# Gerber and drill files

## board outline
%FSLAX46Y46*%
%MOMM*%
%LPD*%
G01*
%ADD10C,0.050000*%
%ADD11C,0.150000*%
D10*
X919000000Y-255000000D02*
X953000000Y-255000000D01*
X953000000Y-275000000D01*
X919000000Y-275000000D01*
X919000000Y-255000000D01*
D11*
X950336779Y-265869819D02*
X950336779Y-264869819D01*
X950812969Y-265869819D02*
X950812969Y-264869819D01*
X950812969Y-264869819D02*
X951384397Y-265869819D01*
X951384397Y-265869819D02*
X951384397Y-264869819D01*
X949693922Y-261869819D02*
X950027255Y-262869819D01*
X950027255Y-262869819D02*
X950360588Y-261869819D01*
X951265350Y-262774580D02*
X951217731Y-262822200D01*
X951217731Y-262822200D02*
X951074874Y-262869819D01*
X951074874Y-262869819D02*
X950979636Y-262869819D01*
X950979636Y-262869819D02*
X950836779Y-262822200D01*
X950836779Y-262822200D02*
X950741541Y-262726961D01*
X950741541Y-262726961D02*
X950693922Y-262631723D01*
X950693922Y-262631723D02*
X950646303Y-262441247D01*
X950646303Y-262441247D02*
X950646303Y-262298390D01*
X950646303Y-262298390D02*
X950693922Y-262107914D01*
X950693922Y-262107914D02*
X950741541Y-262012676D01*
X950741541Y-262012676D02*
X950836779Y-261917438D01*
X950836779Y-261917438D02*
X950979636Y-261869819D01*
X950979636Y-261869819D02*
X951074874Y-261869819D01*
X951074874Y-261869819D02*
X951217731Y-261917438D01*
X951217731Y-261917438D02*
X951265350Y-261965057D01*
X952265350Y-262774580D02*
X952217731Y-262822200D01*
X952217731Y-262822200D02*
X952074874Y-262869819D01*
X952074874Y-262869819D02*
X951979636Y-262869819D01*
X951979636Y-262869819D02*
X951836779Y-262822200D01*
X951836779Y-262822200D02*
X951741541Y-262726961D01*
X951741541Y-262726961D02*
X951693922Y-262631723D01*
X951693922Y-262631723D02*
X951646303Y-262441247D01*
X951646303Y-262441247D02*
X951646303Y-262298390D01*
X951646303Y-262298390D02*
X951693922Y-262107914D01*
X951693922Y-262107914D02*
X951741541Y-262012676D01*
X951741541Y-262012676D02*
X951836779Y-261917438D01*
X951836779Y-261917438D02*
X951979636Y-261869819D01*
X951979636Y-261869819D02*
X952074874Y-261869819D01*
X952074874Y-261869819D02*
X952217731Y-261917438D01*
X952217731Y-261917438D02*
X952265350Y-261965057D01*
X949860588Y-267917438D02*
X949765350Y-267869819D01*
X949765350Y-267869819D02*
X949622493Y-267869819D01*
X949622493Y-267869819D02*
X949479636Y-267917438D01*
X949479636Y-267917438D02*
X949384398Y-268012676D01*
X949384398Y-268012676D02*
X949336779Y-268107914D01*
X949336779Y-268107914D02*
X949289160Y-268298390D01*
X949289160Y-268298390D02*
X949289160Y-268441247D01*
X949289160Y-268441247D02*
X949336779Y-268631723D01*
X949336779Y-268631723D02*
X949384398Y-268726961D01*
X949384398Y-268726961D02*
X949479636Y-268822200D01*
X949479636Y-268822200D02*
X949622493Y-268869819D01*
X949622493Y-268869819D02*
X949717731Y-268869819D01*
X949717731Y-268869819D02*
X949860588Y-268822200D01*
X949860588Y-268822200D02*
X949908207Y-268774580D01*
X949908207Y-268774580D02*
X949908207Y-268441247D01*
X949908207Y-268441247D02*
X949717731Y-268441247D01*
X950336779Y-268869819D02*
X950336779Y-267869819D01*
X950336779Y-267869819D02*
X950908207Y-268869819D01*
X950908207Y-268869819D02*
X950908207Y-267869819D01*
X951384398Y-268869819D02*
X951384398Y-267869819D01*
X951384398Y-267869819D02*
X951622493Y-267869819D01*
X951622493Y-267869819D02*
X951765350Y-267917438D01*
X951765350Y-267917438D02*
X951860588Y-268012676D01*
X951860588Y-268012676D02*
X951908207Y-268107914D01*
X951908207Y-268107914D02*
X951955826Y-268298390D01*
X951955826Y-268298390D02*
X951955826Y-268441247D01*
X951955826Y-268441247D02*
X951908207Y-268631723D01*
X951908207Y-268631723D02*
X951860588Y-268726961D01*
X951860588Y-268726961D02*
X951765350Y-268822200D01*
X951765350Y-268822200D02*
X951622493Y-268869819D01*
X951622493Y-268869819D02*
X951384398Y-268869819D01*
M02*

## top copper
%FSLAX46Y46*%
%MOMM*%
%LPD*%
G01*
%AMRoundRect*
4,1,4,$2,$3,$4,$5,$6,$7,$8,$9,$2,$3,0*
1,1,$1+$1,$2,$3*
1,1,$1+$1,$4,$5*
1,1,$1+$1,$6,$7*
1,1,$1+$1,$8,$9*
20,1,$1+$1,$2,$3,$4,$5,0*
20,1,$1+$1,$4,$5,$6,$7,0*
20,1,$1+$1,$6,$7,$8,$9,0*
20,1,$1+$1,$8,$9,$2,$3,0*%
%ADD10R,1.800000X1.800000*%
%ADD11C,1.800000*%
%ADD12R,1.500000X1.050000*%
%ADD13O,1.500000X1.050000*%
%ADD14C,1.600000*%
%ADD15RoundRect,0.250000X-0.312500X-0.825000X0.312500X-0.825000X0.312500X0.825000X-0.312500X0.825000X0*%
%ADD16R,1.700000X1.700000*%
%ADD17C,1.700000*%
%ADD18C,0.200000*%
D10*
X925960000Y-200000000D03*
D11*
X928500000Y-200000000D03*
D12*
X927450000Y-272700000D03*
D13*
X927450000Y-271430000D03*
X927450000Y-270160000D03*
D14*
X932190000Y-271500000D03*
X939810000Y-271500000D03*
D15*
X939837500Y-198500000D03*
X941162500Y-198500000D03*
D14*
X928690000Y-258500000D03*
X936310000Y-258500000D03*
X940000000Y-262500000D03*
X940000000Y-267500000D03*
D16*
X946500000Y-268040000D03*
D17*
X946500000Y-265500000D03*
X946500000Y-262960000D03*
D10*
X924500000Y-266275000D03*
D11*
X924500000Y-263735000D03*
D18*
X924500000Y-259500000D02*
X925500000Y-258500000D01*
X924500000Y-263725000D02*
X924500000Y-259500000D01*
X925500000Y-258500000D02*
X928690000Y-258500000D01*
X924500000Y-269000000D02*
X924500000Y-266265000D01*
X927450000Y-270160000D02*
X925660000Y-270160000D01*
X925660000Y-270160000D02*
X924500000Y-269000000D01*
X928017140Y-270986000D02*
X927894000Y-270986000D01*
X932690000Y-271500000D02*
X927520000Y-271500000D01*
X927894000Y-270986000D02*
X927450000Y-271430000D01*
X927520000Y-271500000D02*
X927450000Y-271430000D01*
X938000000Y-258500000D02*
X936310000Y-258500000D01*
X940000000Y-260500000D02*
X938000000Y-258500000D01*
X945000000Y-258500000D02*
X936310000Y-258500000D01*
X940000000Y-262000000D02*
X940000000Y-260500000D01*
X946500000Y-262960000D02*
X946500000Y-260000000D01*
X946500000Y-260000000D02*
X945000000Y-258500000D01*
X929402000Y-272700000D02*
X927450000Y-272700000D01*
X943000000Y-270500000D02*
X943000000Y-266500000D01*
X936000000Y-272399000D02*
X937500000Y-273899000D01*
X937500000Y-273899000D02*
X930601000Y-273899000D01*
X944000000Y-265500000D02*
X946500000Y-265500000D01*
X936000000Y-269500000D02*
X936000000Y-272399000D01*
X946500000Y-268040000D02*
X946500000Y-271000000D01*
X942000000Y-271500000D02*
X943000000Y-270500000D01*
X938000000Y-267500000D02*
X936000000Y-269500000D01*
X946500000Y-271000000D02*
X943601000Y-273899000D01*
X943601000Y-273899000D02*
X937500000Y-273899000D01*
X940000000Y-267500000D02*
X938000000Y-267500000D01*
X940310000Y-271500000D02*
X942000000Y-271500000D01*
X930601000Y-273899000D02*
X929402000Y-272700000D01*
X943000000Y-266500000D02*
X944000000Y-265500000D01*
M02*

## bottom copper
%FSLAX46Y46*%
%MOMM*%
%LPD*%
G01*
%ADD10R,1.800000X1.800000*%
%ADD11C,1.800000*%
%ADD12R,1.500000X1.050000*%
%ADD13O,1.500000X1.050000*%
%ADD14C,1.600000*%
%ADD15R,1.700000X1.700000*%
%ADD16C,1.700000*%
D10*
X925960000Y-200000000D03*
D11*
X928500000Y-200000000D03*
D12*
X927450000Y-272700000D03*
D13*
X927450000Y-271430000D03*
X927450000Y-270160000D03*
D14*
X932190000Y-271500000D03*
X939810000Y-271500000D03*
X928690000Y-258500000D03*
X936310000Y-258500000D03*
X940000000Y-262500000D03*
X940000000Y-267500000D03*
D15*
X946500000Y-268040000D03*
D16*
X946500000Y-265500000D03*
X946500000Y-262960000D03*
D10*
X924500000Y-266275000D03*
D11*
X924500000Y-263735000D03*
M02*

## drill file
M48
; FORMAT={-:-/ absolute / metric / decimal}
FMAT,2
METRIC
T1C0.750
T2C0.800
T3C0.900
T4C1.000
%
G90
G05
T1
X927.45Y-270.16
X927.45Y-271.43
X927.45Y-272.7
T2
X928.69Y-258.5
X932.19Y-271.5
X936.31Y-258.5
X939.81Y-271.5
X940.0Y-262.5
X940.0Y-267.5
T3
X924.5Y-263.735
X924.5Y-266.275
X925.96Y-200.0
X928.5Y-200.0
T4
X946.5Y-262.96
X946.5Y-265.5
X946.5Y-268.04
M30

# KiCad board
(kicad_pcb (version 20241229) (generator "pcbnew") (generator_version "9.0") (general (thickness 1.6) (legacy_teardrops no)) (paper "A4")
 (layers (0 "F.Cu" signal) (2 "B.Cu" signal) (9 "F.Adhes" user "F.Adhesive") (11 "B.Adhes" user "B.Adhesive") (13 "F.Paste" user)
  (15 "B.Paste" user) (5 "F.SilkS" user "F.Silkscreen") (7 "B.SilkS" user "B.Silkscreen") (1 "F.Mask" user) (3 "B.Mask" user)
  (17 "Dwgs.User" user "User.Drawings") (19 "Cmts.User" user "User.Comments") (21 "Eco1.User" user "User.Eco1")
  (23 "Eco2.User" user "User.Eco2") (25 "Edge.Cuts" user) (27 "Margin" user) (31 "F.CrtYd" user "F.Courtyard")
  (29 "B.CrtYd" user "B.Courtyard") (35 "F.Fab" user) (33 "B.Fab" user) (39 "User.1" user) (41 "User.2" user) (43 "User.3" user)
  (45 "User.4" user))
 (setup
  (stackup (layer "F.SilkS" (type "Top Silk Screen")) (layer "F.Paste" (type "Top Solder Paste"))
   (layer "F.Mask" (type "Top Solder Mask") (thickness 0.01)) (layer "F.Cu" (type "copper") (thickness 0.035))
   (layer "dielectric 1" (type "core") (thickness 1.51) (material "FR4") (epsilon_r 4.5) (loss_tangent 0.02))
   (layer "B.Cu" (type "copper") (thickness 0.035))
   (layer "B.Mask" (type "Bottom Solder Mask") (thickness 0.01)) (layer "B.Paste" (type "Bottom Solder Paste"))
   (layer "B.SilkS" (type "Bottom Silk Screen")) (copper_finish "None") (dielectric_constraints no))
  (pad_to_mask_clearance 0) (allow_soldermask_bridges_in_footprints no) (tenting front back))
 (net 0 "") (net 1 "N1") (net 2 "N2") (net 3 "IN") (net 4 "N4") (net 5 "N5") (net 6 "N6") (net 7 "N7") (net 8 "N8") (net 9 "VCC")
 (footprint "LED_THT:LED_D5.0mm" (layer "F.Cu") (at 925.96 200)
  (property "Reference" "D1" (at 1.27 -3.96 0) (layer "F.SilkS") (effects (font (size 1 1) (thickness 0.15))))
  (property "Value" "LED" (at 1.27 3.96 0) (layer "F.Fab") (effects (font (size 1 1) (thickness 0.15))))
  (pad "1" thru_hole rect (at 0 0) (size 1.8 1.8) (drill 0.9) (layers "*.Cu" "*.Mask") (remove_unused_layers no) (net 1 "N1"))
  (pad "2" thru_hole circle (at 2.54 0) (size 1.8 1.8) (drill 0.9) (layers "*.Cu" "*.Mask") (remove_unused_layers no) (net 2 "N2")))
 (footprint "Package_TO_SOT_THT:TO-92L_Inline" (layer "F.Cu") (at 927.45 272.7 90)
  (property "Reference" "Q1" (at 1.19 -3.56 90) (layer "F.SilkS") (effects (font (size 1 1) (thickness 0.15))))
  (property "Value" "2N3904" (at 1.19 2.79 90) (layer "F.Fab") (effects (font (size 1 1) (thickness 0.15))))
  (pad "1" thru_hole rect (at 0 0 90) (size 1.05 1.5) (drill 0.75) (layers "*.Cu" "*.Mask") (remove_unused_layers no) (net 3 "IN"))
  (pad "2" thru_hole oval (at 1.27 0 90) (size 1.05 1.5) (drill 0.75) (layers "*.Cu" "*.Mask") (remove_unused_layers no) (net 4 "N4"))
  (pad "3" thru_hole oval (at 2.54 0 90) (size 1.05 1.5) (drill 0.75) (layers "*.Cu" "*.Mask") (remove_unused_layers no) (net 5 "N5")))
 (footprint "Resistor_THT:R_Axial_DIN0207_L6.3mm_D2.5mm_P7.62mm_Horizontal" (layer "F.Cu") (at 932.19 271.5)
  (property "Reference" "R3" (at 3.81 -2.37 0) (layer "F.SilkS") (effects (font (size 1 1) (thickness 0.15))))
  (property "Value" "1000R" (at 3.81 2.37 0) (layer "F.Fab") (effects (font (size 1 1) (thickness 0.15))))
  (pad "1" thru_hole circle (at 0 0) (size 1.6 1.6) (drill 0.8) (layers "*.Cu" "*.Mask") (remove_unused_layers no) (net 4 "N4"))
  (pad "2" thru_hole circle (at 7.62 0) (size 1.6 1.6) (drill 0.8) (layers "*.Cu" "*.Mask") (remove_unused_layers no) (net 3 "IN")))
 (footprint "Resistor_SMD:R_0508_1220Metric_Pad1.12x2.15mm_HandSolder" (layer "F.Cu") (at 940.5 198.5)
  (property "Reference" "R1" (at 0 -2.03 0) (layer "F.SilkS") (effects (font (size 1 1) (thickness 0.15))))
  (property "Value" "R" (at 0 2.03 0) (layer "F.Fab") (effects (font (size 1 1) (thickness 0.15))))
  (pad "1" smd roundrect (at -0.6625 0) (size 1.125 2.15) (layers "F.Cu" "F.Mask" "F.Paste") (roundrect_rratio 0.222222) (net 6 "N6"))
  (pad "2" smd roundrect (at 0.6625 0) (size 1.125 2.15) (layers "F.Cu" "F.Mask" "F.Paste") (roundrect_rratio 0.222222) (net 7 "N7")))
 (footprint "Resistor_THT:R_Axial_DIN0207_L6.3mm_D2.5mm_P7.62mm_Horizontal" (layer "F.Cu") (at 928.69 258.5)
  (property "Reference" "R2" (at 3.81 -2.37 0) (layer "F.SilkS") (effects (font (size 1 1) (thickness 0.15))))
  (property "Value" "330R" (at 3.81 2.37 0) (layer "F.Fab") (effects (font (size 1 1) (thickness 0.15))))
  (pad "1" thru_hole circle (at 0 0) (size 1.6 1.6) (drill 0.8) (layers "*.Cu" "*.Mask") (remove_unused_layers no) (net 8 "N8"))
  (pad "2" thru_hole circle (at 7.62 0) (size 1.6 1.6) (drill 0.8) (layers "*.Cu" "*.Mask") (remove_unused_layers no) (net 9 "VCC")))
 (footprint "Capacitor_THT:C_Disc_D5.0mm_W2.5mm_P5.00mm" (layer "F.Cu") (at 940 262.5 -90)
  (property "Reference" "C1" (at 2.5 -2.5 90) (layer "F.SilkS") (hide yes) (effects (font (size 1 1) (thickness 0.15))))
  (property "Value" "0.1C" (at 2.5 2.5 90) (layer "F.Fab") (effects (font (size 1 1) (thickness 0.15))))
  (pad "1" thru_hole circle (at 0 0 270) (size 1.6 1.6) (drill 0.8) (layers "*.Cu" "*.Mask") (remove_unused_layers no) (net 9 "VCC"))
  (pad "2" thru_hole circle (at 5 0 270) (size 1.6 1.6) (drill 0.8) (layers "*.Cu" "*.Mask") (remove_unused_layers no) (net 3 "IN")))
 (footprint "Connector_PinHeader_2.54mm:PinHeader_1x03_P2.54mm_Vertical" (layer "F.Cu") (at 946.5 268.04 180)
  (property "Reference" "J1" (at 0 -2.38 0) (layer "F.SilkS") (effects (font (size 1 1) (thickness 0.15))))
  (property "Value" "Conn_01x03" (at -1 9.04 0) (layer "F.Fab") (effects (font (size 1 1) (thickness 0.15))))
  (pad "1" thru_hole rect (at 0 0 180) (size 1.7 1.7) (drill 1) (layers "*.Cu" "*.Mask") (remove_unused_layers no) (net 3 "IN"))
  (pad "2" thru_hole circle (at 0 2.54 180) (size 1.7 1.7) (drill 1) (layers "*.Cu" "*.Mask") (remove_unused_layers no) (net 3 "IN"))
  (pad "3" thru_hole circle (at 0 5.08 180) (size 1.7 1.7) (drill 1) (layers "*.Cu" "*.Mask") (remove_unused_layers no) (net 9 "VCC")))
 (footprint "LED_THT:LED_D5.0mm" (layer "F.Cu") (at 924.5 266.275 90)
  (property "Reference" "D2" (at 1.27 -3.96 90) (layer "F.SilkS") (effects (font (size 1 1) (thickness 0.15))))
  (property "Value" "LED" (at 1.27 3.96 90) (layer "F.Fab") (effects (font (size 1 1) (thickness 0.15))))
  (pad "1" thru_hole rect (at 0 0 90) (size 1.8 1.8) (drill 0.9) (layers "*.Cu" "*.Mask") (remove_unused_layers no) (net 5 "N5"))
  (pad "2" thru_hole circle (at 2.54 0 90) (size 1.8 1.8) (drill 0.9) (layers "*.Cu" "*.Mask") (remove_unused_layers no) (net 8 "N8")))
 (gr_rect (start 919 255) (end 953 275) (stroke (width 0.05) (type solid)) (fill no) (layer "Edge.Cuts"))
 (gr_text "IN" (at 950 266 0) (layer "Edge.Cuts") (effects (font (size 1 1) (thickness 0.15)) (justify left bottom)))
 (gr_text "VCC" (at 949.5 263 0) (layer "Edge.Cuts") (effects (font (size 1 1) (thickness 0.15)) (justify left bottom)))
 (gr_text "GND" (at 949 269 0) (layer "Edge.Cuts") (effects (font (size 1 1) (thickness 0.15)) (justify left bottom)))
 (segment (start 924.5 259.5) (end 925.5 258.5) (width 0.2) (layer "F.Cu") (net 8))
 (segment (start 924.5 263.725) (end 924.5 259.5) (width 0.2) (layer "F.Cu") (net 8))
 (segment (start 925.5 258.5) (end 928.69 258.5) (width 0.2) (layer "F.Cu") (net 8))
 (segment (start 924.5 269) (end 924.5 266.265) (width 0.2) (layer "F.Cu") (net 5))
 (segment (start 927.45 270.16) (end 925.66 270.16) (width 0.2) (layer "F.Cu") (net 5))
 (segment (start 925.66 270.16) (end 924.5 269) (width 0.2) (layer "F.Cu") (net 5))
 (segment (start 928.01714 270.986) (end 927.894 270.986) (width 0.2) (layer "F.Cu") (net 4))
 (segment (start 932.69 271.5) (end 927.52 271.5) (width 0.2) (layer "F.Cu") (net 4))
 (segment (start 927.894 270.986) (end 927.45 271.43) (width 0.2) (layer "F.Cu") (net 4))
 (segment (start 927.52 271.5) (end 927.45 271.43) (width 0.2) (layer "F.Cu") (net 4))
 (segment (start 938 258.5) (end 936.31 258.5) (width 0.2) (layer "F.Cu") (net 9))
 (segment (start 940 260.5) (end 938 258.5) (width 0.2) (layer "F.Cu") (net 9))
 (segment (start 945 258.5) (end 936.31 258.5) (width 0.2) (layer "F.Cu") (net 9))
 (segment (start 940 262) (end 940 260.5) (width 0.2) (layer "F.Cu") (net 9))
 (segment (start 946.5 262.96) (end 946.5 260) (width 0.2) (layer "F.Cu") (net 9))
 (segment (start 946.5 260) (end 945 258.5) (width 0.2) (layer "F.Cu") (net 9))
 (segment (start 929.402 272.7) (end 927.45 272.7) (width 0.2) (layer "F.Cu") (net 3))
 (segment (start 943 270.5) (end 943 266.5) (width 0.2) (layer "F.Cu") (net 3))
 (segment (start 936 272.399) (end 937.5 273.899) (width 0.2) (layer "F.Cu") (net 3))
 (segment (start 937.5 273.899) (end 930.601 273.899) (width 0.2) (layer "F.Cu") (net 3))
 (segment (start 944 265.5) (end 946.5 265.5) (width 0.2) (layer "F.Cu") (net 3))
 (segment (start 936 269.5) (end 936 272.399) (width 0.2) (layer "F.Cu") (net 3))
 (segment (start 946.5 268.04) (end 946.5 271) (width 0.2) (layer "F.Cu") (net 3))
 (segment (start 942 271.5) (end 943 270.5) (width 0.2) (layer "F.Cu") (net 3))
 (segment (start 938 267.5) (end 936 269.5) (width 0.2) (layer "F.Cu") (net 3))
 (segment (start 946.5 271) (end 943.601 273.899) (width 0.2) (layer "F.Cu") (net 3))
 (segment (start 943.601 273.899) (end 937.5 273.899) (width 0.2) (layer "F.Cu") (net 3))
 (segment (start 940 267.5) (end 938 267.5) (width 0.2) (layer "F.Cu") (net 3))
 (segment (start 940.31 271.5) (end 942 271.5) (width 0.2) (layer "F.Cu") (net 3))
 (segment (start 930.601 273.899) (end 929.402 272.7) (width 0.2) (layer "F.Cu") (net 3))
 (segment (start 943 266.5) (end 944 265.5) (width 0.2) (layer "F.Cu") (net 3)))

